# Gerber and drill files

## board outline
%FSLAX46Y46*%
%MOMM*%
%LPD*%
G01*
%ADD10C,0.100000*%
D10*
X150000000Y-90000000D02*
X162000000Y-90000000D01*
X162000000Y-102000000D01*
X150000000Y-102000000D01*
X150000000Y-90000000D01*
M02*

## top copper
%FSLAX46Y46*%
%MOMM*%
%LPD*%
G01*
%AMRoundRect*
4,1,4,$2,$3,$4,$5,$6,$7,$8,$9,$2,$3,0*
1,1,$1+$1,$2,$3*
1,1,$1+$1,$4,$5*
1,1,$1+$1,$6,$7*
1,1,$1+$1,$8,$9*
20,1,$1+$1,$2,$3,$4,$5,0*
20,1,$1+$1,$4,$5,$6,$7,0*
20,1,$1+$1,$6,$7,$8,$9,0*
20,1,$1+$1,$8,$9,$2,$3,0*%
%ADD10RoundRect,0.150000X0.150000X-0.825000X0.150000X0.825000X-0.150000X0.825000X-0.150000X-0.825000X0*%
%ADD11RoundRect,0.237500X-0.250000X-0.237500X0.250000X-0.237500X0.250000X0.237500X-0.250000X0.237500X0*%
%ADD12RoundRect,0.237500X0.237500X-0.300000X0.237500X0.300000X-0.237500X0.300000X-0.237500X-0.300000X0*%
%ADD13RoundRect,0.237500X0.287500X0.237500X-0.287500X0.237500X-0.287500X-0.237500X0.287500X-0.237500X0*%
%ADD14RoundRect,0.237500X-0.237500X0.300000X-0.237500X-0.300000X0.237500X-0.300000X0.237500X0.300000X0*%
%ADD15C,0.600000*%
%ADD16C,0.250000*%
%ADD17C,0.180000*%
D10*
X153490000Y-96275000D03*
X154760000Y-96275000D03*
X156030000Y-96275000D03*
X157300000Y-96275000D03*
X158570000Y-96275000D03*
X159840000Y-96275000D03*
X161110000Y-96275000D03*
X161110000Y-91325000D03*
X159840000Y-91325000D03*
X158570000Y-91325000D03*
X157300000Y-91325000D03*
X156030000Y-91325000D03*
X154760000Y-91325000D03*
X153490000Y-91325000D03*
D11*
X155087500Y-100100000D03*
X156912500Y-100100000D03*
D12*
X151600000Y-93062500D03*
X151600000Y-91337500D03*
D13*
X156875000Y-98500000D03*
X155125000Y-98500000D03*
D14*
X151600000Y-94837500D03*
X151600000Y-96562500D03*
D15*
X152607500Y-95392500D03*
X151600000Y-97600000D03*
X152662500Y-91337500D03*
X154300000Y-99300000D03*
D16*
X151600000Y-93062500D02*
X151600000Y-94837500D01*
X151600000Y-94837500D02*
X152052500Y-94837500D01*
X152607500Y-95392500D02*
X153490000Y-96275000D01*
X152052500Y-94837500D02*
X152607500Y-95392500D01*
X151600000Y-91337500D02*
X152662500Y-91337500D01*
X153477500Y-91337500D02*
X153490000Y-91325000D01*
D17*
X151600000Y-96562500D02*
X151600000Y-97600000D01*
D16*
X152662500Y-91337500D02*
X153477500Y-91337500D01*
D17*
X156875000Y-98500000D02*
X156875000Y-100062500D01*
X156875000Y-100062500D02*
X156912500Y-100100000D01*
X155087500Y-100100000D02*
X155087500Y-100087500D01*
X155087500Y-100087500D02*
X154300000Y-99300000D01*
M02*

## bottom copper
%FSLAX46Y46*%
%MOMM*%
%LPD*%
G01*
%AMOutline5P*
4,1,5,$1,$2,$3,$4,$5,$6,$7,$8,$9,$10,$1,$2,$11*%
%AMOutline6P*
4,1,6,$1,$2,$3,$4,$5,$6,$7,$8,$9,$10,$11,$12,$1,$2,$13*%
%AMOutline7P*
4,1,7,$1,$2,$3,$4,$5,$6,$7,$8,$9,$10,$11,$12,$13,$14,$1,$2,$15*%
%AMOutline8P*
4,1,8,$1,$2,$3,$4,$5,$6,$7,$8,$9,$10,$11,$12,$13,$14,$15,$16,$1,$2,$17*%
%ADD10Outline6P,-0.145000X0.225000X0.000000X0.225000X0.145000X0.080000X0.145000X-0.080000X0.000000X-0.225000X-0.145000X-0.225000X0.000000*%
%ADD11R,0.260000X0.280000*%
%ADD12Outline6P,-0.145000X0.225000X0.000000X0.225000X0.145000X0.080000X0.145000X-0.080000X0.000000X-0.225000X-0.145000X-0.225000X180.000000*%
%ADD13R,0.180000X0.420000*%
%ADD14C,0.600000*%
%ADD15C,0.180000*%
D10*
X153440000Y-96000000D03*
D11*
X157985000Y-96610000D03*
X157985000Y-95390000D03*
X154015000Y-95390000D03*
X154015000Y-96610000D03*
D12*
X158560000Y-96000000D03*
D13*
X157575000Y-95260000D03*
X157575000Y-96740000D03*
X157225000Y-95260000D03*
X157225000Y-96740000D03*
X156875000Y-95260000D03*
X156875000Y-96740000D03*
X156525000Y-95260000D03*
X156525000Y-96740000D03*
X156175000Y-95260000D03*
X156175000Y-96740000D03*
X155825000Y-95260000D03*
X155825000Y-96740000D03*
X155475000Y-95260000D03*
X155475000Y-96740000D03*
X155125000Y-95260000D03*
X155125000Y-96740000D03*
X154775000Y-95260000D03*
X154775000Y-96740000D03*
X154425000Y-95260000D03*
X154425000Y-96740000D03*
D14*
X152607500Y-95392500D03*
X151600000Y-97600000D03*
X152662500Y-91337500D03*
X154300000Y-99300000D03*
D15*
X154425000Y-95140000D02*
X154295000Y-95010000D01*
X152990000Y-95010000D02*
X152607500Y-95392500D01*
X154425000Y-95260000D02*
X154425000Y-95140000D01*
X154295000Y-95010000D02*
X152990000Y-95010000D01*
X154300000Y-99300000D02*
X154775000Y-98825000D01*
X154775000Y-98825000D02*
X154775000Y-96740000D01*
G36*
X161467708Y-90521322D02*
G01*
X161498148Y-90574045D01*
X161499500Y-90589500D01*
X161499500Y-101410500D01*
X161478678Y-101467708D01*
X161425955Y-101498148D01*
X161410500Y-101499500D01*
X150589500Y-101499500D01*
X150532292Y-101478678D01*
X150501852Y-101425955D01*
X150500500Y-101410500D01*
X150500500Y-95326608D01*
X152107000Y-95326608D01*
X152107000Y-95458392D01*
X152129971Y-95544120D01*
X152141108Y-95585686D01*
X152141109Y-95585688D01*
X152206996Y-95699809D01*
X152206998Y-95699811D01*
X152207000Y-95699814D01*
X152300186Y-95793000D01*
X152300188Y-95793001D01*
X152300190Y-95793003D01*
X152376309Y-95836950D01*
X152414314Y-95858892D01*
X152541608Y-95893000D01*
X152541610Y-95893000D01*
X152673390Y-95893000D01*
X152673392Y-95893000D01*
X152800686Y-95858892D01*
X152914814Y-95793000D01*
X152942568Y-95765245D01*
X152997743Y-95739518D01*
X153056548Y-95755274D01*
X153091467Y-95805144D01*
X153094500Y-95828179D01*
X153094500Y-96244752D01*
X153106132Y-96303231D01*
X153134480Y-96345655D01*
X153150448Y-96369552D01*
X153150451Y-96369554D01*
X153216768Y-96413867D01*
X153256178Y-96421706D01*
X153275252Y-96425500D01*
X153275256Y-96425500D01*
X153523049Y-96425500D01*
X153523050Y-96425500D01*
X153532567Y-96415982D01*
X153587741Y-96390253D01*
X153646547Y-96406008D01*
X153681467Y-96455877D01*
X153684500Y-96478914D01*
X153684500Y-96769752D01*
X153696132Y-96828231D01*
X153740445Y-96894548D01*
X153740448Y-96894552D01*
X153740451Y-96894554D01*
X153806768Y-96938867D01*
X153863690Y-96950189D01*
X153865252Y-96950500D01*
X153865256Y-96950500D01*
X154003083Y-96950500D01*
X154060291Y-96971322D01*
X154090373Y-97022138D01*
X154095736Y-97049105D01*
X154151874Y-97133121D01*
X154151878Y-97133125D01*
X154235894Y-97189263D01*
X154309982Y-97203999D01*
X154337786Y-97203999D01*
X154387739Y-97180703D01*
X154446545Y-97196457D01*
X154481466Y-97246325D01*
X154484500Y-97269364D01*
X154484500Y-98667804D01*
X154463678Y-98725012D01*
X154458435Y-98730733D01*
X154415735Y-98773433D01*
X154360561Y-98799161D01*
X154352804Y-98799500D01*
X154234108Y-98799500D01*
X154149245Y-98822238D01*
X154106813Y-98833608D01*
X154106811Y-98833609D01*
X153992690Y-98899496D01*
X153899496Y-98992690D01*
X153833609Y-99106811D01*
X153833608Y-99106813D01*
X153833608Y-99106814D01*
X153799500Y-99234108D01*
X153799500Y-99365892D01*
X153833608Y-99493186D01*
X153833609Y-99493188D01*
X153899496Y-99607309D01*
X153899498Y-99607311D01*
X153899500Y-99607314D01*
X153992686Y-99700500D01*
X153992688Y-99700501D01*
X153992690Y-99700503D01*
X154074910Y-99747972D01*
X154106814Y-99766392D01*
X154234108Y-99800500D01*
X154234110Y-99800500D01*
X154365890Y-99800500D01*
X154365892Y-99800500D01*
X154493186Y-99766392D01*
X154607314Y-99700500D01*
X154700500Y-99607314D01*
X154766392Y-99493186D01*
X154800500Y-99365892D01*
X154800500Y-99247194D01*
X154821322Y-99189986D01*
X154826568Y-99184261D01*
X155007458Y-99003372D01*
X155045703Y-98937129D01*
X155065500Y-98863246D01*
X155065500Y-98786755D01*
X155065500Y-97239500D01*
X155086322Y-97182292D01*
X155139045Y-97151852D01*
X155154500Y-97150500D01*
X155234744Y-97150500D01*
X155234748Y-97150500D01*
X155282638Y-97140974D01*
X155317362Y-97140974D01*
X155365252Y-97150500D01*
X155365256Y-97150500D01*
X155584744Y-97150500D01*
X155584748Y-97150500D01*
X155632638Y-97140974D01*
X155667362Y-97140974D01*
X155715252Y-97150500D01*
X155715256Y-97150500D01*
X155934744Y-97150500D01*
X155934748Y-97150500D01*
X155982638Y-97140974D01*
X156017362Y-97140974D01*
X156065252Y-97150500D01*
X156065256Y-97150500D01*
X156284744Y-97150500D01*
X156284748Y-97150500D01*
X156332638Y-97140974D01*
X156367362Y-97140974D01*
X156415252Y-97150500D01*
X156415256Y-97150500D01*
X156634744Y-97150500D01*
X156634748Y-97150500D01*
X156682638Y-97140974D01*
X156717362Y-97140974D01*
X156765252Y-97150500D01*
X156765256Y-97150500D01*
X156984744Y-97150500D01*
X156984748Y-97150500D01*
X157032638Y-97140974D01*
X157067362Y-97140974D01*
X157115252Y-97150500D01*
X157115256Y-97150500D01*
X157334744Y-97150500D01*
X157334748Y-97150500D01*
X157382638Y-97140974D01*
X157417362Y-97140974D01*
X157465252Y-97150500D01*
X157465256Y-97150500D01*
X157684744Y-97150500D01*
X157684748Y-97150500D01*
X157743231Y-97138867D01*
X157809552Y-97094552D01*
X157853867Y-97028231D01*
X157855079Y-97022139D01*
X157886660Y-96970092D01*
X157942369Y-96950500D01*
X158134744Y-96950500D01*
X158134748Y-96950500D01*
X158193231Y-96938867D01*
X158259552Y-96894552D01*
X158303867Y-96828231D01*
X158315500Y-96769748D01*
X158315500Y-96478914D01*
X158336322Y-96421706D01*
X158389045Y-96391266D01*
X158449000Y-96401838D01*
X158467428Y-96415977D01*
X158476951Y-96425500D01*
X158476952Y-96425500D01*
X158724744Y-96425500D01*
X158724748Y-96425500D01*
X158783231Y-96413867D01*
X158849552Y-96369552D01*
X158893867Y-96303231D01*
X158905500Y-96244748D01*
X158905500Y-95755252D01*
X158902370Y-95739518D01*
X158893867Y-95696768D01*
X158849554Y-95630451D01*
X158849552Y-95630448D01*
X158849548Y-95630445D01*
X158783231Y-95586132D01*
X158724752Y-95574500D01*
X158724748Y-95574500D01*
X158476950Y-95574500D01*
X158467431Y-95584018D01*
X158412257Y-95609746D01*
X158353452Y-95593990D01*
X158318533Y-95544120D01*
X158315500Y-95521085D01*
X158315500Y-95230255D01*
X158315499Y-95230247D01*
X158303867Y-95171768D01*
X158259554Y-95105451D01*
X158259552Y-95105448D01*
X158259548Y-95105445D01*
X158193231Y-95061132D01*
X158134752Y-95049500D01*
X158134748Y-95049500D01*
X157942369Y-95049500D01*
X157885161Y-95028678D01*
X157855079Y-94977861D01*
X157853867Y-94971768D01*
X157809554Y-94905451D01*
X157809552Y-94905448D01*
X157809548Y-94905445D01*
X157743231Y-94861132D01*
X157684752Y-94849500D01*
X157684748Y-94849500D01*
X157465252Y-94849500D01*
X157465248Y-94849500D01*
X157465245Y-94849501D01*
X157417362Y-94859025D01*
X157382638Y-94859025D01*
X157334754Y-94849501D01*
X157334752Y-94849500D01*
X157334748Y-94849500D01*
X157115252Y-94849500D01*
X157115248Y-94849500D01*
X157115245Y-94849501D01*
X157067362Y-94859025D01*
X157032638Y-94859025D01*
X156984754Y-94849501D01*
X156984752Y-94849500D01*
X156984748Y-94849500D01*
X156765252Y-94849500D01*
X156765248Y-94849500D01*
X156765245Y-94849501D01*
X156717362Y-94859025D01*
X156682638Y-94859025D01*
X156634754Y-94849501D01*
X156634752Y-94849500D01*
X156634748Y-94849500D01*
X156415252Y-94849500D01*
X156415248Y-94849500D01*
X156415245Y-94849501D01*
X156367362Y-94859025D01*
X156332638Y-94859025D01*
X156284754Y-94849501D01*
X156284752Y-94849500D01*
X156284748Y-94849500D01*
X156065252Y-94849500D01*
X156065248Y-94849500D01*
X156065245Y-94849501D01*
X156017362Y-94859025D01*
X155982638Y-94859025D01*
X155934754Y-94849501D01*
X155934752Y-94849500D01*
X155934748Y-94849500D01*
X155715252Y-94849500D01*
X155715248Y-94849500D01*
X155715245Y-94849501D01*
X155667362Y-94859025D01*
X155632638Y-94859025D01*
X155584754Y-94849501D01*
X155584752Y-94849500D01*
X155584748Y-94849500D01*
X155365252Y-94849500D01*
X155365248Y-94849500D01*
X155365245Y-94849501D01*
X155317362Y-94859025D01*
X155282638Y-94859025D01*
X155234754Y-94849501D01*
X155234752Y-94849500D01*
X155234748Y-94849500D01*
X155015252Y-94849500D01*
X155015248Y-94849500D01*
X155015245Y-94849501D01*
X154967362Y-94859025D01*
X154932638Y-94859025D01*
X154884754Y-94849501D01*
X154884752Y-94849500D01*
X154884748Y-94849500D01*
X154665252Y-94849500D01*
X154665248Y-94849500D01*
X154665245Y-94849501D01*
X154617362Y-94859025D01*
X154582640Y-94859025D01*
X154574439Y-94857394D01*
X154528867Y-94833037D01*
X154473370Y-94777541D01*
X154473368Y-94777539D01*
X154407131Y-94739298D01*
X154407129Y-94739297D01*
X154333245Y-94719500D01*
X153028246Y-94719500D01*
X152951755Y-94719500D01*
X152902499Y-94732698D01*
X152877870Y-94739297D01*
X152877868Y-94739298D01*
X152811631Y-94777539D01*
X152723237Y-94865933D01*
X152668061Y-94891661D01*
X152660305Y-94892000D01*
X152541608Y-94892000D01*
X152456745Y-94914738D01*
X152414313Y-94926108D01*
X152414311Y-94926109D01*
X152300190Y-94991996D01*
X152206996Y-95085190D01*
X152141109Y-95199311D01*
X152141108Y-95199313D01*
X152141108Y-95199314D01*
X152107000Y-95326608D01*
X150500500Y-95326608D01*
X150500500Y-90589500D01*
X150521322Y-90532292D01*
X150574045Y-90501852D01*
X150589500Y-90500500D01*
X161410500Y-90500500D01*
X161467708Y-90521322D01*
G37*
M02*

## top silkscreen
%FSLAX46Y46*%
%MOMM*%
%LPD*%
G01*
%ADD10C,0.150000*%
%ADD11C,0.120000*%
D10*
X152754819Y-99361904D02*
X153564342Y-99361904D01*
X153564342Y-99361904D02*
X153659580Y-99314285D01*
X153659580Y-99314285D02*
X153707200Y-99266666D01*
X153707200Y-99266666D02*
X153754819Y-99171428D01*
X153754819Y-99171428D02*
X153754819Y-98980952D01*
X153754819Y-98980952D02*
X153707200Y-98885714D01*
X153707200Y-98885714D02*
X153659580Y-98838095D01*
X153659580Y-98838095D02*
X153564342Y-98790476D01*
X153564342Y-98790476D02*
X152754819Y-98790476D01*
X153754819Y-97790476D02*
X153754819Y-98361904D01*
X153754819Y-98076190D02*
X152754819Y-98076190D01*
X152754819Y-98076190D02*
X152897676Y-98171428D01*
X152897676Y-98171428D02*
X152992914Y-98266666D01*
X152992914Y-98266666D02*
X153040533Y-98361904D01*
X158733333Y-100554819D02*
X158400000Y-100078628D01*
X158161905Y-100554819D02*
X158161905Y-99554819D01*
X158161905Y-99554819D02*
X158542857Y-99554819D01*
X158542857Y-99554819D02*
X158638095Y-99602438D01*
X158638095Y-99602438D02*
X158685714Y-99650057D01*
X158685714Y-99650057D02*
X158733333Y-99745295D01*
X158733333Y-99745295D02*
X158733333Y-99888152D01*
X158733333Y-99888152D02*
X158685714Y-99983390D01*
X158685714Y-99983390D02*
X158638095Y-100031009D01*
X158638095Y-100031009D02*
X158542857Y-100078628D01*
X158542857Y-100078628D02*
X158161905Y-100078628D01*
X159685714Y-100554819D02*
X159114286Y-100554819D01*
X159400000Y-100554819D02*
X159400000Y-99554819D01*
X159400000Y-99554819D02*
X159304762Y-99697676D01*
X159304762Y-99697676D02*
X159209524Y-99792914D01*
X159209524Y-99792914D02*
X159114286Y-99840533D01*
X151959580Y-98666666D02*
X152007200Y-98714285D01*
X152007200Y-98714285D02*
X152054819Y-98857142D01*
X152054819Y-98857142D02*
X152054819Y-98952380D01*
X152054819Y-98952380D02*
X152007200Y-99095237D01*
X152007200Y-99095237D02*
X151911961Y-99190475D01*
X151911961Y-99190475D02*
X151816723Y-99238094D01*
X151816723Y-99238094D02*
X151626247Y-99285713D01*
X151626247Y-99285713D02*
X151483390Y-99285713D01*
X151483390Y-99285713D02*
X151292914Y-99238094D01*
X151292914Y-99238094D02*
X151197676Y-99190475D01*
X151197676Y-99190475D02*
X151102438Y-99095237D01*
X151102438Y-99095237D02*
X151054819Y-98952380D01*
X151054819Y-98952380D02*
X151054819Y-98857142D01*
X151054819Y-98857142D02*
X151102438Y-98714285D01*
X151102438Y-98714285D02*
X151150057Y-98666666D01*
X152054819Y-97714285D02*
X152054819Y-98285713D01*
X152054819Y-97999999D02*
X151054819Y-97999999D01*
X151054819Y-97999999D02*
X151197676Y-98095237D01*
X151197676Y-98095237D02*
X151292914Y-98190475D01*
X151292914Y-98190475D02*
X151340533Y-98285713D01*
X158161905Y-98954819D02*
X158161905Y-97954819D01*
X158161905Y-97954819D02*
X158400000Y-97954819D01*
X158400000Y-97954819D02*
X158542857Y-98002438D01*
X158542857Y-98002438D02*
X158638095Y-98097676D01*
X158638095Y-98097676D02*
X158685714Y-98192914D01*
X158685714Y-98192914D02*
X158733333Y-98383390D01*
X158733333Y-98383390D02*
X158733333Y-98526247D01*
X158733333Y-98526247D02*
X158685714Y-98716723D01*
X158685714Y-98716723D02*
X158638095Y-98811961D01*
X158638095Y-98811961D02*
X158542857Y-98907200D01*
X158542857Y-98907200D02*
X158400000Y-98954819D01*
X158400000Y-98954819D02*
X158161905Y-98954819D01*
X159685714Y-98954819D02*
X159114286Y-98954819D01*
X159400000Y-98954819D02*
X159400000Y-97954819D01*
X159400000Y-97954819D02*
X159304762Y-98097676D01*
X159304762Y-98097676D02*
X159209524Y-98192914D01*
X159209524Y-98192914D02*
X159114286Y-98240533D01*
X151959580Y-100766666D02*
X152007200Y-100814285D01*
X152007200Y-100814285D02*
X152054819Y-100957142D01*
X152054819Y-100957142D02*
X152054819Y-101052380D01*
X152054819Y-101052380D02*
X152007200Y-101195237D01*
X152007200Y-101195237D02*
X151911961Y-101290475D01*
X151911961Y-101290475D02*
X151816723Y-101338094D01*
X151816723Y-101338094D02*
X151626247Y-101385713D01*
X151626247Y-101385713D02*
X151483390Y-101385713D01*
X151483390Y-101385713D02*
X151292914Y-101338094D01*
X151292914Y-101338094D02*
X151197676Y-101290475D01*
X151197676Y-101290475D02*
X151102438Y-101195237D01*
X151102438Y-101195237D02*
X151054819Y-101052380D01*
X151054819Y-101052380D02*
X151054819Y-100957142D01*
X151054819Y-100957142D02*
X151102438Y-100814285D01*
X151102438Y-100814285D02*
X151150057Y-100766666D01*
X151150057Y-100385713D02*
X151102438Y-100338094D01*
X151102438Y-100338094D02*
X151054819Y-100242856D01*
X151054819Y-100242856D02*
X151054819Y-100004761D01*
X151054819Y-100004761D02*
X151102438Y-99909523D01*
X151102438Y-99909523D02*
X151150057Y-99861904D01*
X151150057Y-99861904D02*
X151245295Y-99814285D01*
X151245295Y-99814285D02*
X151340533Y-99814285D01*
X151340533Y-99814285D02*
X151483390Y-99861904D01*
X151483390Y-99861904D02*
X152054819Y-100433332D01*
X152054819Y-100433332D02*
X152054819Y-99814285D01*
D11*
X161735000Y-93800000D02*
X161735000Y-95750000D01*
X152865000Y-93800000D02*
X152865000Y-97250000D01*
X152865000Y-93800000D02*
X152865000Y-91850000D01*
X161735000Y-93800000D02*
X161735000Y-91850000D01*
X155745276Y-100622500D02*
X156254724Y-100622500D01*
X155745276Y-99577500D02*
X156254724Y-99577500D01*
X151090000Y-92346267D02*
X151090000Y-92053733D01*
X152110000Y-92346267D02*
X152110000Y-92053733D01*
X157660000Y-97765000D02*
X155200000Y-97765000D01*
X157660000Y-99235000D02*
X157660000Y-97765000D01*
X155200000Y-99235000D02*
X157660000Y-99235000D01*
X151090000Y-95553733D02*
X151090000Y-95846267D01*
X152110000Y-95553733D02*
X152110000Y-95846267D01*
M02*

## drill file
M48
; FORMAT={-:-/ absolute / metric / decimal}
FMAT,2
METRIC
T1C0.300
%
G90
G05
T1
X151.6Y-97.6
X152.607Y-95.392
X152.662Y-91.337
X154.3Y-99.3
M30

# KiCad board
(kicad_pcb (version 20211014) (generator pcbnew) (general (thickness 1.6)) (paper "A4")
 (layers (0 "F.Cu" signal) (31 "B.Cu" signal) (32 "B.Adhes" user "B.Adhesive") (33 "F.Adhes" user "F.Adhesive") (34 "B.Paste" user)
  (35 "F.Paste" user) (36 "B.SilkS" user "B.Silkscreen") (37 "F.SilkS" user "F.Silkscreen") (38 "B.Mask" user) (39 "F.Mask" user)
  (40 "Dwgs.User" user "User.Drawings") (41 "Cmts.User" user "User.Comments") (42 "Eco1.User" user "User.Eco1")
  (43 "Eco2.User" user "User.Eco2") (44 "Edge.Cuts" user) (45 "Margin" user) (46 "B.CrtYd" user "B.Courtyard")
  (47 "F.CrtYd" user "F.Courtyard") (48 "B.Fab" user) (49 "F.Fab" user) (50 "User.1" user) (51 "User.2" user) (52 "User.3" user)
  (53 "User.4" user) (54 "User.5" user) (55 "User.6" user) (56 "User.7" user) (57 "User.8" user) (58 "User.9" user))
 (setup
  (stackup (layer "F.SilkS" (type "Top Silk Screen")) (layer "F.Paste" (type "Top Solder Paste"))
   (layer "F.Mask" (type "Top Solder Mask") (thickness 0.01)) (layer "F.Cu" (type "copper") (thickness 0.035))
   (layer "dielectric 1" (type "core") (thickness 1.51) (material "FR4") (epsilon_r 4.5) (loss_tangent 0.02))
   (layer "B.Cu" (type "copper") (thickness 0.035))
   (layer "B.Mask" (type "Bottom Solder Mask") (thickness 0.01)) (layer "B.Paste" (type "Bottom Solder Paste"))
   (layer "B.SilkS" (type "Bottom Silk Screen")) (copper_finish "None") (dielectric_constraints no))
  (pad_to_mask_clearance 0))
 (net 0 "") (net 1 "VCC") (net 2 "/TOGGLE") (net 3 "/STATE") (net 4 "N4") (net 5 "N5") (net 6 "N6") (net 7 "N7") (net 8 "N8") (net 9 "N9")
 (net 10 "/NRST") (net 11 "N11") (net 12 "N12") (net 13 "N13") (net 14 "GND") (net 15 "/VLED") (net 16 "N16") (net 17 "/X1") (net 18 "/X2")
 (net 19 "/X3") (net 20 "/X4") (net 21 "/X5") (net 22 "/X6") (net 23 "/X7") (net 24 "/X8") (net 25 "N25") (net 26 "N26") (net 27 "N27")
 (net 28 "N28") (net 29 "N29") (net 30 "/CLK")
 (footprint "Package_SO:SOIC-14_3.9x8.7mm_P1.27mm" (layer "F.Cu") (at 157.3 93.8 90)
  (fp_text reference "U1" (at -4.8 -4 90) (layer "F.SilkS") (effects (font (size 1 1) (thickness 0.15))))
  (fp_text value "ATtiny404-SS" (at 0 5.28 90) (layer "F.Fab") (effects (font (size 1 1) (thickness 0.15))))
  (fp_line (start 0 4.435) (end -1.95 4.435) (layer "F.SilkS") (width 0.12))
  (fp_line (start 0 -4.435) (end -3.45 -4.435) (layer "F.SilkS") (width 0.12))
  (fp_line (start 0 -4.435) (end 1.95 -4.435) (layer "F.SilkS") (width 0.12))
  (fp_line (start 0 4.435) (end 1.95 4.435) (layer "F.SilkS") (width 0.12))
  (pad "1" smd roundrect (at -2.475 -3.81 90) (size 1.95 0.6) (layers "F.Cu" "F.Paste" "F.Mask") (roundrect_rratio 0.25) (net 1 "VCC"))
  (pad "2" smd roundrect (at -2.475 -2.54 90) (size 1.95 0.6) (layers "F.Cu" "F.Paste" "F.Mask") (roundrect_rratio 0.25) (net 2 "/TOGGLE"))
  (pad "3" smd roundrect (at -2.475 -1.27 90) (size 1.95 0.6) (layers "F.Cu" "F.Paste" "F.Mask") (roundrect_rratio 0.25) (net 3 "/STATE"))
  (pad "4" smd roundrect (at -2.475 0 90) (size 1.95 0.6) (layers "F.Cu" "F.Paste" "F.Mask") (roundrect_rratio 0.25) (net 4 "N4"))
  (pad "5" smd roundrect (at -2.475 1.27 90) (size 1.95 0.6) (layers "F.Cu" "F.Paste" "F.Mask") (roundrect_rratio 0.25) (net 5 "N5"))
  (pad "6" smd roundrect (at -2.475 2.54 90) (size 1.95 0.6) (layers "F.Cu" "F.Paste" "F.Mask") (roundrect_rratio 0.25) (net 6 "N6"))
  (pad "7" smd roundrect (at -2.475 3.81 90) (size 1.95 0.6) (layers "F.Cu" "F.Paste" "F.Mask") (roundrect_rratio 0.25) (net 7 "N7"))
  (pad "8" smd roundrect (at 2.475 3.81 90) (size 1.95 0.6) (layers "F.Cu" "F.Paste" "F.Mask") (roundrect_rratio 0.25) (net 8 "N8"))
  (pad "9" smd roundrect (at 2.475 2.54 90) (size 1.95 0.6) (layers "F.Cu" "F.Paste" "F.Mask") (roundrect_rratio 0.25) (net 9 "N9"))
  (pad "10" smd roundrect (at 2.475 1.27 90) (size 1.95 0.6) (layers "F.Cu" "F.Paste" "F.Mask") (roundrect_rratio 0.25) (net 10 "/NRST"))
  (pad "11" smd roundrect (at 2.475 0 90) (size 1.95 0.6) (layers "F.Cu" "F.Paste" "F.Mask") (roundrect_rratio 0.25) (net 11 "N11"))
  (pad "12" smd roundrect (at 2.475 -1.27 90) (size 1.95 0.6) (layers "F.Cu" "F.Paste" "F.Mask") (roundrect_rratio 0.25) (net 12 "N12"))
  (pad "13" smd roundrect (at 2.475 -2.54 90) (size 1.95 0.6) (layers "F.Cu" "F.Paste" "F.Mask") (roundrect_rratio 0.25) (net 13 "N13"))
  (pad "14" smd roundrect (at 2.475 -3.81 90) (size 1.95 0.6) (layers "F.Cu" "F.Paste" "F.Mask") (roundrect_rratio 0.25) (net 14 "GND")))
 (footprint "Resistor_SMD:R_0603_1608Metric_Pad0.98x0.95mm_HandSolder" (layer "F.Cu") (at 156 100.1)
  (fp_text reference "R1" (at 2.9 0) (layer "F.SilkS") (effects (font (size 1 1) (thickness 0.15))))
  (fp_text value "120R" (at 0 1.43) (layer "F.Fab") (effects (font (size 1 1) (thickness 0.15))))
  (fp_line (start -0.254724 0.5225) (end 0.254724 0.5225) (layer "F.SilkS") (width 0.12))
  (fp_line (start -0.254724 -0.5225) (end 0.254724 -0.5225) (layer "F.SilkS") (width 0.12))
  (pad "1" smd roundrect (at -0.9125 0) (size 0.975 0.95) (layers "F.Cu" "F.Paste" "F.Mask") (roundrect_rratio 0.25) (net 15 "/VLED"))
  (pad "2" smd roundrect (at 0.9125 0) (size 0.975 0.95) (layers "F.Cu" "F.Paste" "F.Mask") (roundrect_rratio 0.25) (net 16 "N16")))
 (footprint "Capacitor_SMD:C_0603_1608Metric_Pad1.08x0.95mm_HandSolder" (layer "F.Cu") (at 151.6 92.2 90)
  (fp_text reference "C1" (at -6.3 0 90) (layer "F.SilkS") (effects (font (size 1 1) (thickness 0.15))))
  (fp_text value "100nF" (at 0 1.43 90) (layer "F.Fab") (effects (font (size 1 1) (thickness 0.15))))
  (fp_line (start -0.146267 -0.51) (end 0.146267 -0.51) (layer "F.SilkS") (width 0.12))
  (fp_line (start -0.146267 0.51) (end 0.146267 0.51) (layer "F.SilkS") (width 0.12))
  (pad "1" smd roundrect (at -0.8625 0 90) (size 1.075 0.95) (layers "F.Cu" "F.Paste" "F.Mask") (roundrect_rratio 0.25) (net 1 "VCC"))
  (pad "2" smd roundrect (at 0.8625 0 90) (size 1.075 0.95) (layers "F.Cu" "F.Paste" "F.Mask") (roundrect_rratio 0.25) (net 14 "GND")))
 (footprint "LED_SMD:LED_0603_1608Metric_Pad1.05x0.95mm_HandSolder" (layer "F.Cu") (at 156 98.5 180)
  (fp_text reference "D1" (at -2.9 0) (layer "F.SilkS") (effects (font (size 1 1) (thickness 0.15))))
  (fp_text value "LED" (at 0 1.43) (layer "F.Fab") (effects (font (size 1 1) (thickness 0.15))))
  (fp_line (start -1.66 0.735) (end 0.8 0.735) (layer "F.SilkS") (width 0.12))
  (fp_line (start -1.66 -0.735) (end -1.66 0.735) (layer "F.SilkS") (width 0.12))
  (fp_line (start 0.8 -0.735) (end -1.66 -0.735) (layer "F.SilkS") (width 0.12))
  (pad "1" smd roundrect (at -0.875 0 180) (size 1.05 0.95) (layers "F.Cu" "F.Paste" "F.Mask") (roundrect_rratio 0.25) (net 16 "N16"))
  (pad "2" smd roundrect (at 0.875 0 180) (size 1.05 0.95) (layers "F.Cu" "F.Paste" "F.Mask") (roundrect_rratio 0.25) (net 3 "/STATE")))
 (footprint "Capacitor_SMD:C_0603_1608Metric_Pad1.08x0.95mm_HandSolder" (layer "F.Cu") (at 151.6 95.7 -90)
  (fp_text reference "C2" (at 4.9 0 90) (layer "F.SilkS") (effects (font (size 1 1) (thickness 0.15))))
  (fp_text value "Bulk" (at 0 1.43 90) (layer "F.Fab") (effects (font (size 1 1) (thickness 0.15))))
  (fp_line (start -0.146267 0.51) (end 0.146267 0.51) (layer "F.SilkS") (width 0.12))
  (fp_line (start -0.146267 -0.51) (end 0.146267 -0.51) (layer "F.SilkS") (width 0.12))
  (pad "1" smd roundrect (at -0.8625 0 270) (size 1.075 0.95) (layers "F.Cu" "F.Paste" "F.Mask") (roundrect_rratio 0.25) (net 1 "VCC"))
  (pad "2" smd roundrect (at 0.8625 0 270) (size 1.075 0.95) (layers "F.Cu" "F.Paste" "F.Mask") (roundrect_rratio 0.25) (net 14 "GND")))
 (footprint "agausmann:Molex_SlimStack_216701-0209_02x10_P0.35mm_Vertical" (layer "B.Cu") (at 156 96 180)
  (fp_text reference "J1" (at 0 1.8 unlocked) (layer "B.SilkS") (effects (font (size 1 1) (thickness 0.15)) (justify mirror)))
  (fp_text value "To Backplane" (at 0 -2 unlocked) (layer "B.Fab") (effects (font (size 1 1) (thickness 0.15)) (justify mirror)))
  (pad "" smd roundrect (at 2.56 0) (size 0.29 0.45) (layers "B.Cu" "B.Paste" "B.Mask") (roundrect_rratio 0) (chamfer_ratio 0.5)
   (chamfer top_right bottom_right))
  (pad "" smd rect (at -1.985 -0.61 180) (size 0.26 0.28) (layers "B.Cu" "B.Paste" "B.Mask"))
  (pad "" smd rect (at -1.985 0.61 180) (size 0.26 0.28) (layers "B.Cu" "B.Paste" "B.Mask"))
  (pad "" smd rect (at 1.985 0.61 180) (size 0.26 0.28) (layers "B.Cu" "B.Paste" "B.Mask"))
  (pad "" smd rect (at 1.985 -0.61 180) (size 0.26 0.28) (layers "B.Cu" "B.Paste" "B.Mask"))
  (pad "" smd roundrect (at -2.56 0 180) (size 0.29 0.45) (layers "B.Cu" "B.Paste" "B.Mask") (roundrect_rratio 0) (chamfer_ratio 0.5)
   (chamfer top_right bottom_right))
  (pad "1" smd rect (at -1.575 0.74 180) (size 0.18 0.42) (layers "B.Cu" "B.Paste" "B.Mask") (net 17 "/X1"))
  (pad "2" smd rect (at -1.575 -0.74 180) (size 0.18 0.42) (layers "B.Cu" "B.Paste" "B.Mask") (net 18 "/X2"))
  (pad "3" smd rect (at -1.225 0.74 180) (size 0.18 0.42) (layers "B.Cu" "B.Paste" "B.Mask") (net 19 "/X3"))
  (pad "4" smd rect (at -1.225 -0.74 180) (size 0.18 0.42) (layers "B.Cu" "B.Paste" "B.Mask") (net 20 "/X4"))
  (pad "5" smd rect (at -0.875 0.74 180) (size 0.18 0.42) (layers "B.Cu" "B.Paste" "B.Mask") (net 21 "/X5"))
  (pad "6" smd rect (at -0.875 -0.74 180) (size 0.18 0.42) (layers "B.Cu" "B.Paste" "B.Mask") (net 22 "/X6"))
  (pad "7" smd rect (at -0.525 0.74 180) (size 0.18 0.42) (layers "B.Cu" "B.Paste" "B.Mask") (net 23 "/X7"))
  (pad "8" smd rect (at -0.525 -0.74 180) (size 0.18 0.42) (layers "B.Cu" "B.Paste" "B.Mask") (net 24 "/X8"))
  (pad "9" smd rect (at -0.175 0.74 180) (size 0.18 0.42) (layers "B.Cu" "B.Paste" "B.Mask") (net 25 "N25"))
  (pad "10" smd rect (at -0.175 -0.74 180) (size 0.18 0.42) (layers "B.Cu" "B.Paste" "B.Mask") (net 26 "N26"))
  (pad "11" smd rect (at 0.175 0.74 180) (size 0.18 0.42) (layers "B.Cu" "B.Paste" "B.Mask") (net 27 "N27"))
  (pad "12" smd rect (at 0.175 -0.74 180) (size 0.18 0.42) (layers "B.Cu" "B.Paste" "B.Mask") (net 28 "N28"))
  (pad "13" smd rect (at 0.525 0.74 180) (size 0.18 0.42) (layers "B.Cu" "B.Paste" "B.Mask") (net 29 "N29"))
  (pad "14" smd rect (at 0.525 -0.74 180) (size 0.18 0.42) (layers "B.Cu" "B.Paste" "B.Mask") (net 3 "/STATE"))
  (pad "15" smd rect (at 0.875 0.74 180) (size 0.18 0.42) (layers "B.Cu" "B.Paste" "B.Mask") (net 10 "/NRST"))
  (pad "16" smd rect (at 0.875 -0.74 180) (size 0.18 0.42) (layers "B.Cu" "B.Paste" "B.Mask") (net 2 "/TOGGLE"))
  (pad "17" smd rect (at 1.225 0.74 180) (size 0.18 0.42) (layers "B.Cu" "B.Paste" "B.Mask") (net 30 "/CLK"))
  (pad "18" smd rect (at 1.225 -0.74 180) (size 0.18 0.42) (layers "B.Cu" "B.Paste" "B.Mask") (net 15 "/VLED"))
  (pad "19" smd rect (at 1.575 0.74 180) (size 0.18 0.42) (layers "B.Cu" "B.Paste" "B.Mask") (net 1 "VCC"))
  (pad "20" smd rect (at 1.575 -0.74 180) (size 0.18 0.42) (layers "B.Cu" "B.Paste" "B.Mask") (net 14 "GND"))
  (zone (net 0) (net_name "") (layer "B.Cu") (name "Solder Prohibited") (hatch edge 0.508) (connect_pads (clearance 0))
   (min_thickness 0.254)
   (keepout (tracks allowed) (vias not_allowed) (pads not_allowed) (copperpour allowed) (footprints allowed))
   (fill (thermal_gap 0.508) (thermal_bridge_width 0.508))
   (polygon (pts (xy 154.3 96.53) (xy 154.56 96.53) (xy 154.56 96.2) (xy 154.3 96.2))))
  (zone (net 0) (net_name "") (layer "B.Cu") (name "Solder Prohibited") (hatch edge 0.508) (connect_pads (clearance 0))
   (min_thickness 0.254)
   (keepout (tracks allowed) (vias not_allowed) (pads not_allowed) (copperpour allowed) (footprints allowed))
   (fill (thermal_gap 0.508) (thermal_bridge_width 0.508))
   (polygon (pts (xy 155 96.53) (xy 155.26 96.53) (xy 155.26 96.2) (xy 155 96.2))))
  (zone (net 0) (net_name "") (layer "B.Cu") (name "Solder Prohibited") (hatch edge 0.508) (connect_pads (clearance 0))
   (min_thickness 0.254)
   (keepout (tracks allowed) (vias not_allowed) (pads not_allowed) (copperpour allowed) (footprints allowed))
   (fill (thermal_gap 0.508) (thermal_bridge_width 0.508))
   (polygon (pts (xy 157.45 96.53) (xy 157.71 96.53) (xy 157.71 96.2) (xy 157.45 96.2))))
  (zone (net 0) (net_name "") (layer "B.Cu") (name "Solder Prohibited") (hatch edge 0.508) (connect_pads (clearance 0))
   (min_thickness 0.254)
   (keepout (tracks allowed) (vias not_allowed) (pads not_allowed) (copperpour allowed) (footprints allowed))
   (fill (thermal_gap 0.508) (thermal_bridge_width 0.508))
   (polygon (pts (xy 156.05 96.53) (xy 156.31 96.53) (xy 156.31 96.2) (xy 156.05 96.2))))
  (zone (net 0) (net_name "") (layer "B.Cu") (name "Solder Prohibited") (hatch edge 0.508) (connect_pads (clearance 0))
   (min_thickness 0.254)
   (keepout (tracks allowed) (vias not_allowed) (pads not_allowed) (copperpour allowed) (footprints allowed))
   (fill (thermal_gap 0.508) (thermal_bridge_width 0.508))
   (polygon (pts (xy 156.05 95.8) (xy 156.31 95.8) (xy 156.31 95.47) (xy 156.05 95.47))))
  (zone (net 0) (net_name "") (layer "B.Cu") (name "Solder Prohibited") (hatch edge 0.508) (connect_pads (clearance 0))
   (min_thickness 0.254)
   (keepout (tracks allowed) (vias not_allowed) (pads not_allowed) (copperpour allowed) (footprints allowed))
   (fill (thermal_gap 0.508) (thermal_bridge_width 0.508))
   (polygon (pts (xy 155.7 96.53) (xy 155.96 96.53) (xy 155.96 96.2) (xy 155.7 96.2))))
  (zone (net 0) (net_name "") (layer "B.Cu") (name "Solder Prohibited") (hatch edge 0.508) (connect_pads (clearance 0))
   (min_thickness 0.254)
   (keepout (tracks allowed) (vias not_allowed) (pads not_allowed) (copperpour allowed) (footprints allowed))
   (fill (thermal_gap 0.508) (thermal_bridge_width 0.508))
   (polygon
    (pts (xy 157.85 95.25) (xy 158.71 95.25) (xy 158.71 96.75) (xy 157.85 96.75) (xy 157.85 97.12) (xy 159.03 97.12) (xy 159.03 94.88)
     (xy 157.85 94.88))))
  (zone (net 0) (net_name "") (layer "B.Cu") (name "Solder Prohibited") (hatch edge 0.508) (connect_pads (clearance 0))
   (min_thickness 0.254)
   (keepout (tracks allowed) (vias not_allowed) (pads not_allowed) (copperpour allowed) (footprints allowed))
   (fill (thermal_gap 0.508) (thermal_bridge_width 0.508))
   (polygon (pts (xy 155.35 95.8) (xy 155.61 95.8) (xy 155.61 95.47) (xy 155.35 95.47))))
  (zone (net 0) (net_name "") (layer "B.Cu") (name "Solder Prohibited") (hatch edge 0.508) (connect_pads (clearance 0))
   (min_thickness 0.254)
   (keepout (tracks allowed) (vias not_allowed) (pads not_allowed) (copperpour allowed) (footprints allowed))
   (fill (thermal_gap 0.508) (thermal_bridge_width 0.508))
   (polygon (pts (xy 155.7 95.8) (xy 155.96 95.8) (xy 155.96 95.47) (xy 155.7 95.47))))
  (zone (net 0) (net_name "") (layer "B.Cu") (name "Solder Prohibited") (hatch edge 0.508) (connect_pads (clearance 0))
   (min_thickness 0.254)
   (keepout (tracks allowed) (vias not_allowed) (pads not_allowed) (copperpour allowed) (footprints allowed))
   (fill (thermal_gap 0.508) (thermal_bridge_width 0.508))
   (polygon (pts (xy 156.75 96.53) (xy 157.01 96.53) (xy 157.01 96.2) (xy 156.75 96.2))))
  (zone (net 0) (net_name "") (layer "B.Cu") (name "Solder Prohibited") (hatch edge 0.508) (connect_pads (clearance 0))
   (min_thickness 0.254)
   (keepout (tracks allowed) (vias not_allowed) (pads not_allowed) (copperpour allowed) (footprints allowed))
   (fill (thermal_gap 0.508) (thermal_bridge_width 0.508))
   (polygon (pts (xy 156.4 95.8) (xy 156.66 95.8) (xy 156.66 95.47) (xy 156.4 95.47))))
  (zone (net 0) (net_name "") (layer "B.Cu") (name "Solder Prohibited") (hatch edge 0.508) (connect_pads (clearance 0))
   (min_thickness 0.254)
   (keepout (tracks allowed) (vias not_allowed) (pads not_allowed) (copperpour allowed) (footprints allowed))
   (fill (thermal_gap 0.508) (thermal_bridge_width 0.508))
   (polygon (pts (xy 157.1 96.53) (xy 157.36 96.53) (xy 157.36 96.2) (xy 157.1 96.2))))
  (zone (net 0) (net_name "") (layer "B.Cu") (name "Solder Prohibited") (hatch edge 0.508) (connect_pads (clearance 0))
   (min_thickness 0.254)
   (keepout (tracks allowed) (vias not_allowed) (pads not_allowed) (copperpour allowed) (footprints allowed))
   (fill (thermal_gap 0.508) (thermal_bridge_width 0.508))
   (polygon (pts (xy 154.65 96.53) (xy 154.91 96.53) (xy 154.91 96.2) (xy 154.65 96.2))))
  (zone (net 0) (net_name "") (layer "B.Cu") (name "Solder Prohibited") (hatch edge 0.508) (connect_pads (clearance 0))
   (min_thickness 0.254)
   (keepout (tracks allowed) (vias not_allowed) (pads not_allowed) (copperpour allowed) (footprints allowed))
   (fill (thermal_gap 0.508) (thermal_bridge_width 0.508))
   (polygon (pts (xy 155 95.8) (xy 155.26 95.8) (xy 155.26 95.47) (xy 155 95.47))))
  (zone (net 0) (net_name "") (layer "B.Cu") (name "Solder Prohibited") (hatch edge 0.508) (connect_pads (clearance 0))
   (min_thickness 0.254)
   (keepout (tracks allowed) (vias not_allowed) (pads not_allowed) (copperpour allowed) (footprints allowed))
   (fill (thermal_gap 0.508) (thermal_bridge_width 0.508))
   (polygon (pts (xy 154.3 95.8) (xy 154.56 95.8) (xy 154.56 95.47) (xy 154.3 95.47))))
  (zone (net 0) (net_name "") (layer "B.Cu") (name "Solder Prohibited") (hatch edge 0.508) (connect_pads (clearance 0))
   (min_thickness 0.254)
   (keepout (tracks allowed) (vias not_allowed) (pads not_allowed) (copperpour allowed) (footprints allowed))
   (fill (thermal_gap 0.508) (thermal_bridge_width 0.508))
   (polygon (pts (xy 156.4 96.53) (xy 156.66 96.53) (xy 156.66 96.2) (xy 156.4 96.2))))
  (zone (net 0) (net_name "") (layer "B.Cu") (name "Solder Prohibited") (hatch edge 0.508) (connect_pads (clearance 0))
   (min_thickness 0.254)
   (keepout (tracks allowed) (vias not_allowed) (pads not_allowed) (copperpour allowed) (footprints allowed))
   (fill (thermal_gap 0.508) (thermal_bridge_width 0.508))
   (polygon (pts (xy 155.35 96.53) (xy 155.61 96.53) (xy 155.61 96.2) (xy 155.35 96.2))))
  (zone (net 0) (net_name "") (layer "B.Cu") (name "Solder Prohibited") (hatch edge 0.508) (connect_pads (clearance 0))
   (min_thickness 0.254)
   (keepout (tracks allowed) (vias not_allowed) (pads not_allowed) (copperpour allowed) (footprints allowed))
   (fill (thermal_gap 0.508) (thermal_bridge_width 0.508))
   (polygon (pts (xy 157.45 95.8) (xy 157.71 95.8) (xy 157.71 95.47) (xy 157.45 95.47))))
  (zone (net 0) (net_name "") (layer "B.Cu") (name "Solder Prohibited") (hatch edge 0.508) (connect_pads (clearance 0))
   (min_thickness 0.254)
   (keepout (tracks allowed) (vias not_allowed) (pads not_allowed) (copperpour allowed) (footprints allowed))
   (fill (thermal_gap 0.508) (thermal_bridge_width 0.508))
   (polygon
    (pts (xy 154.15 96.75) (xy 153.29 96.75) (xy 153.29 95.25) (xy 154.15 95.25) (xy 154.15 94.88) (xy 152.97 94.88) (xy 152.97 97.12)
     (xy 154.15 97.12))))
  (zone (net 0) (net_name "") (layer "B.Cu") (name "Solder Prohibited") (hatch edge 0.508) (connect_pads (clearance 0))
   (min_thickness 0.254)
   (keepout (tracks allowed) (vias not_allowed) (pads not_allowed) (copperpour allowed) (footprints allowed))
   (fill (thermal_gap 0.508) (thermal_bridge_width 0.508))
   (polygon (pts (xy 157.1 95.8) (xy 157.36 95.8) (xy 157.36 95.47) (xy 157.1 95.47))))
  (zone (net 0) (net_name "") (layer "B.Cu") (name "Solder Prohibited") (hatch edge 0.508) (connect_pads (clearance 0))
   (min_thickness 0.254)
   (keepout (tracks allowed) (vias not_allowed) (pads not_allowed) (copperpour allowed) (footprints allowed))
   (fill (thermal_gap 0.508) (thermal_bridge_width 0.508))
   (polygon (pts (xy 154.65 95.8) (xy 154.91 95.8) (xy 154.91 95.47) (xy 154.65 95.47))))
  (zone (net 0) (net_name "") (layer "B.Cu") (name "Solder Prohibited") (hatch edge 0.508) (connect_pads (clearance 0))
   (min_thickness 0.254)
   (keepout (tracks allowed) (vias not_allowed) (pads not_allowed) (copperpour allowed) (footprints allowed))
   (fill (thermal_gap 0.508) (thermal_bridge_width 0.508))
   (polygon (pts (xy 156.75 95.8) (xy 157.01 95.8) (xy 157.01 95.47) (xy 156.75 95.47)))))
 (gr_rect (start 150 90) (end 162 102) (layer "Edge.Cuts") (width 0.1) (fill none))
 (segment (start 151.6 93.0625) (end 151.6 94.8375) (width 0.25) (layer "F.Cu") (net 1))
 (segment (start 151.6 94.8375) (end 152.0525 94.8375) (width 0.25) (layer "F.Cu") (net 1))
 (segment (start 152.6075 95.3925) (end 153.49 96.275) (width 0.25) (layer "F.Cu") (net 1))
 (segment (start 152.0525 94.8375) (end 152.6075 95.3925) (width 0.25) (layer "F.Cu") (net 1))
 (via (at 152.6075 95.3925) (size 0.6) (drill 0.3) (layers "F.Cu" "B.Cu") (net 1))
 (segment (start 154.425 95.14) (end 154.295 95.01) (width 0.18) (layer "B.Cu") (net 1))
 (segment (start 152.99 95.01) (end 152.6075 95.3925) (width 0.18) (layer "B.Cu") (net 1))
 (segment (start 154.425 95.26) (end 154.425 95.14) (width 0.18) (layer "B.Cu") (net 1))
 (segment (start 154.295 95.01) (end 152.99 95.01) (width 0.18) (layer "B.Cu") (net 1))
 (segment (start 151.6 91.3375) (end 152.6625 91.3375) (width 0.25) (layer "F.Cu") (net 14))
 (segment (start 153.4775 91.3375) (end 153.49 91.325) (width 0.25) (layer "F.Cu") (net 14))
 (segment (start 151.6 96.5625) (end 151.6 97.6) (width 0.18) (layer "F.Cu") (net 14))
 (segment (start 152.6625 91.3375) (end 153.4775 91.3375) (width 0.25) (layer "F.Cu") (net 14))
 (via (at 151.6 97.6) (size 0.6) (drill 0.3) (layers "F.Cu" "B.Cu") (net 14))
 (via (at 152.6625 91.3375) (size 0.6) (drill 0.3) (layers "F.Cu" "B.Cu") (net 14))
 (segment (start 156.875 98.5) (end 156.875 100.0625) (width 0.18) (layer "F.Cu") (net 16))
 (segment (start 156.875 100.0625) (end 156.9125 100.1) (width 0.18) (layer "F.Cu") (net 16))
 (segment (start 155.0875 100.1) (end 155.0875 100.0875) (width 0.18) (layer "F.Cu") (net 15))
 (segment (start 155.0875 100.0875) (end 154.3 99.3) (width 0.18) (layer "F.Cu") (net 15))
 (via (at 154.3 99.3) (size 0.6) (drill 0.3) (layers "F.Cu" "B.Cu") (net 15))
 (segment (start 154.3 99.3) (end 154.775 98.825) (width 0.18) (layer "B.Cu") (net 15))
 (segment (start 154.775 98.825) (end 154.775 96.74) (width 0.18) (layer "B.Cu") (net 15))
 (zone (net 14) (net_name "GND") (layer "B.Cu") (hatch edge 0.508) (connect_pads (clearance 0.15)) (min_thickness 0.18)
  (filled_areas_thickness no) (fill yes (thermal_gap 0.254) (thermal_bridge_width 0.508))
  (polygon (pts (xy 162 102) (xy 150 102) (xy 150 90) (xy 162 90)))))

